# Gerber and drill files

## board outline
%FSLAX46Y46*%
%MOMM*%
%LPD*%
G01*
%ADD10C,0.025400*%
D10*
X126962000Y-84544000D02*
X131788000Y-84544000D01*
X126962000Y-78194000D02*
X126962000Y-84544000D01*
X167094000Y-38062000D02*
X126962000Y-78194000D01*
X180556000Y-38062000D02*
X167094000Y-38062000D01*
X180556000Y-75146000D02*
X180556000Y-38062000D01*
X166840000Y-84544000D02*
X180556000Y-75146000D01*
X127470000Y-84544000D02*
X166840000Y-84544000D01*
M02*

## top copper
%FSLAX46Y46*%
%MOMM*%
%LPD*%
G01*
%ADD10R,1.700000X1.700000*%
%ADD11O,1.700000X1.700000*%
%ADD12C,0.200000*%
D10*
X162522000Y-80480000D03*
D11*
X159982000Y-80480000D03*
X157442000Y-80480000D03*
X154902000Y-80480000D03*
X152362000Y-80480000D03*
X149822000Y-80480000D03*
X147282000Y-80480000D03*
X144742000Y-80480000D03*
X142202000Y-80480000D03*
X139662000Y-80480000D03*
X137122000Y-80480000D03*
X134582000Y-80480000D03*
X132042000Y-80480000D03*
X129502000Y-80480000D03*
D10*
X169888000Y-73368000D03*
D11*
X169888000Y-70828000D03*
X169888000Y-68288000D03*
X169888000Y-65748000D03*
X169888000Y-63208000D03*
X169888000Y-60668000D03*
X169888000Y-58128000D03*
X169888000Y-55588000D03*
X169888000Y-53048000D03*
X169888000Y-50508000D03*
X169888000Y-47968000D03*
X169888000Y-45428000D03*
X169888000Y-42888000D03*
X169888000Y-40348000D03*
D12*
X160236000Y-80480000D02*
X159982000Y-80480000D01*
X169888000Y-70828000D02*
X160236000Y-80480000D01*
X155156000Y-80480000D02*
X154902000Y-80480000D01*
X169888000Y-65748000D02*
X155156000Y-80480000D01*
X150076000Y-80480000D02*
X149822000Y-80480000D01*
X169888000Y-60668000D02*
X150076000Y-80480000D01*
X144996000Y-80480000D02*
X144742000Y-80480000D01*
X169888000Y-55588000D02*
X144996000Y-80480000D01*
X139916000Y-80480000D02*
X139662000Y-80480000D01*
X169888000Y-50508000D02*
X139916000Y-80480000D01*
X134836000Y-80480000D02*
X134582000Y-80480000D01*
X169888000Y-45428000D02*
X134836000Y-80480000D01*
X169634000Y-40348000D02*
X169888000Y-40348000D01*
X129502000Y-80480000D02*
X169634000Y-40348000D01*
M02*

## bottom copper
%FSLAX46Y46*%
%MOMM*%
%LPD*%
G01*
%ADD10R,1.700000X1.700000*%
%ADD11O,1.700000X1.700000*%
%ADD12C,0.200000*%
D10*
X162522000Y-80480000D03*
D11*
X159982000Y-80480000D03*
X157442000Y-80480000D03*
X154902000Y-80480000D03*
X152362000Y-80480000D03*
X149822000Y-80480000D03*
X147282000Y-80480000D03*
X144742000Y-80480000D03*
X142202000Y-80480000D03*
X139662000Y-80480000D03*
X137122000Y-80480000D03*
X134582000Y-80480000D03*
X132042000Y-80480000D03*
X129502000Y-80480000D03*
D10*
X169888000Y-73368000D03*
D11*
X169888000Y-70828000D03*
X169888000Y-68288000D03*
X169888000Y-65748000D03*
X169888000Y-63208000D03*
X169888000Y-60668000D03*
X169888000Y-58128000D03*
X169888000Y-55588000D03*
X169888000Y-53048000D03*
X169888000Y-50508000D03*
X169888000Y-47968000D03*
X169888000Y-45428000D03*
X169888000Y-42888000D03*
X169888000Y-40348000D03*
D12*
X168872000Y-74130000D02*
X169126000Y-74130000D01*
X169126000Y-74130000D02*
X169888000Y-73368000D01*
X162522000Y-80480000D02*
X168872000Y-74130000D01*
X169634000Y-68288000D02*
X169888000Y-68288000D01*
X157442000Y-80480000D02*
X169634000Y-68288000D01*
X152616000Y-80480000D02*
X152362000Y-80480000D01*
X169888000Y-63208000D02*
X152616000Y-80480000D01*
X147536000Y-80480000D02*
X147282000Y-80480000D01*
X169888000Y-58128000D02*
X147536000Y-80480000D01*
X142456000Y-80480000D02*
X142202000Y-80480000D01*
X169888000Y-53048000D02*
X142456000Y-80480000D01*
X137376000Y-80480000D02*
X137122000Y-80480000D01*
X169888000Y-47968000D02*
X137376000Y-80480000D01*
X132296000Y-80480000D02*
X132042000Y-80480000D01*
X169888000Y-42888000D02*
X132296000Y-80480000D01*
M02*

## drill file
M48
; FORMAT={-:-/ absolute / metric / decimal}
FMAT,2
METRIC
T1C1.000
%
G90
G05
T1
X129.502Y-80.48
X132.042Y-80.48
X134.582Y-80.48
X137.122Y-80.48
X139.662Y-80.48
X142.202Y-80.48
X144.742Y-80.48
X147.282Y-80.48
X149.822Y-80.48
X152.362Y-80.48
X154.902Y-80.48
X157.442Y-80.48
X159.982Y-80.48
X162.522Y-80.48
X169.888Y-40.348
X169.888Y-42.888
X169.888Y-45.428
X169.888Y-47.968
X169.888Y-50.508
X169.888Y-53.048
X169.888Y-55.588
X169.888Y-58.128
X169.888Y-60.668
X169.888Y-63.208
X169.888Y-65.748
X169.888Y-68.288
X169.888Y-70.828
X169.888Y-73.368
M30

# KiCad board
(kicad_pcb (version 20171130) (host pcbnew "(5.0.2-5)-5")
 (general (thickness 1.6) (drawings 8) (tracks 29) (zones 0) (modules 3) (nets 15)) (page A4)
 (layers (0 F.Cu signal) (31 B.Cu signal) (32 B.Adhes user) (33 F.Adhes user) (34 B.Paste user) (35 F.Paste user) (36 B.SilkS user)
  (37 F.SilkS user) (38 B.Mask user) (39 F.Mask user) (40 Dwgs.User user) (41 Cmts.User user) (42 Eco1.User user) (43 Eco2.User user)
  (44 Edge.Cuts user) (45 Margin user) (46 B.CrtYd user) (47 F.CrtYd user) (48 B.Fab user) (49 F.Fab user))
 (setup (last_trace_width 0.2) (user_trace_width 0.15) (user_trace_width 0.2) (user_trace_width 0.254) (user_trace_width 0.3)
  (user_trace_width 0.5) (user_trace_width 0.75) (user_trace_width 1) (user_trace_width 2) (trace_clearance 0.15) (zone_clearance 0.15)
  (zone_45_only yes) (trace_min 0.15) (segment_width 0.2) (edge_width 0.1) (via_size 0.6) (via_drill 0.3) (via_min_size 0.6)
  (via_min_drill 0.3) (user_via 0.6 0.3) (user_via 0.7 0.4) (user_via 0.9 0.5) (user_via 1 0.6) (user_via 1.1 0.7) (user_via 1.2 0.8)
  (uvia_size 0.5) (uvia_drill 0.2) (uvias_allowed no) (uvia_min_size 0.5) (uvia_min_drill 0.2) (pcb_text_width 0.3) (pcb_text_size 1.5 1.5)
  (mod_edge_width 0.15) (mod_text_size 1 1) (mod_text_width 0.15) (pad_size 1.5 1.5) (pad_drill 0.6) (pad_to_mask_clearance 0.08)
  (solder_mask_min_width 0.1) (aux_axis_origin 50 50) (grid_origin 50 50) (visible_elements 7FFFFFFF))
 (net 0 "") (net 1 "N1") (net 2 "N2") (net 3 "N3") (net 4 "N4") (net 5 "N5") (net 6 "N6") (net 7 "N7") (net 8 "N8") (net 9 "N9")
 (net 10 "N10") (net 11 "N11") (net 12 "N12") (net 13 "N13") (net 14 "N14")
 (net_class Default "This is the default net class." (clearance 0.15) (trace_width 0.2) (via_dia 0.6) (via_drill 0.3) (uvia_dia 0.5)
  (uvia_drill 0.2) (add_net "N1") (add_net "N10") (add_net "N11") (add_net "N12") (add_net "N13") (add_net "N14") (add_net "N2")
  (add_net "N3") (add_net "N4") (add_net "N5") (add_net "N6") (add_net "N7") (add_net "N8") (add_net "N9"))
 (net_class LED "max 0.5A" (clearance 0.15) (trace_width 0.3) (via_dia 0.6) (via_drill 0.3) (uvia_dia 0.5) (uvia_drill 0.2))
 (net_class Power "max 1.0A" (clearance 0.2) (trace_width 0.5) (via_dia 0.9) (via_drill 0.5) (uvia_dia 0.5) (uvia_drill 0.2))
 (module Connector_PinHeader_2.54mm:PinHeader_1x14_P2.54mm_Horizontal (layer F.Cu) (at 162.522 80.48 270)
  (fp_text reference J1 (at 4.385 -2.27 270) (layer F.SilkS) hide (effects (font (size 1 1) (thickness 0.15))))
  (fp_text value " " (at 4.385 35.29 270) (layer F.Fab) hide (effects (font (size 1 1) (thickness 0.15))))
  (pad 1 thru_hole rect (at 0 0 270) (size 1.7 1.7) (drill 1) (layers *.Cu *.Mask) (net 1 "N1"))
  (pad 2 thru_hole oval (at 0 2.54 270) (size 1.7 1.7) (drill 1) (layers *.Cu *.Mask) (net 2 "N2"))
  (pad 3 thru_hole oval (at 0 5.08 270) (size 1.7 1.7) (drill 1) (layers *.Cu *.Mask) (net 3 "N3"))
  (pad 4 thru_hole oval (at 0 7.62 270) (size 1.7 1.7) (drill 1) (layers *.Cu *.Mask) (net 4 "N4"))
  (pad 5 thru_hole oval (at 0 10.16 270) (size 1.7 1.7) (drill 1) (layers *.Cu *.Mask) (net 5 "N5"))
  (pad 6 thru_hole oval (at 0 12.7 270) (size 1.7 1.7) (drill 1) (layers *.Cu *.Mask) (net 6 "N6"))
  (pad 7 thru_hole oval (at 0 15.24 270) (size 1.7 1.7) (drill 1) (layers *.Cu *.Mask) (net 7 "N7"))
  (pad 8 thru_hole oval (at 0 17.78 270) (size 1.7 1.7) (drill 1) (layers *.Cu *.Mask) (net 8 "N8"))
  (pad 9 thru_hole oval (at 0 20.32 270) (size 1.7 1.7) (drill 1) (layers *.Cu *.Mask) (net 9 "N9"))
  (pad 10 thru_hole oval (at 0 22.86 270) (size 1.7 1.7) (drill 1) (layers *.Cu *.Mask) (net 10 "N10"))
  (pad 11 thru_hole oval (at 0 25.4 270) (size 1.7 1.7) (drill 1) (layers *.Cu *.Mask) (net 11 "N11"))
  (pad 12 thru_hole oval (at 0 27.94 270) (size 1.7 1.7) (drill 1) (layers *.Cu *.Mask) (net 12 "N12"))
  (pad 13 thru_hole oval (at 0 30.48 270) (size 1.7 1.7) (drill 1) (layers *.Cu *.Mask) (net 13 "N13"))
  (pad 14 thru_hole oval (at 0 33.02 270) (size 1.7 1.7) (drill 1) (layers *.Cu *.Mask) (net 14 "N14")))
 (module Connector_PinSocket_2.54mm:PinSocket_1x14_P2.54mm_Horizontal (layer F.Cu) (at 169.888 73.368 180)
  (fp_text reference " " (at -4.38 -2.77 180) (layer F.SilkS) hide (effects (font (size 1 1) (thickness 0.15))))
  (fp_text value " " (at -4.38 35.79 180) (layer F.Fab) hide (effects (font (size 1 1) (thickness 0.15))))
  (pad 1 thru_hole rect (at 0 0 180) (size 1.7 1.7) (drill 1) (layers *.Cu *.Mask) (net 1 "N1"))
  (pad 2 thru_hole oval (at 0 2.54 180) (size 1.7 1.7) (drill 1) (layers *.Cu *.Mask) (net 2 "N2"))
  (pad 3 thru_hole oval (at 0 5.08 180) (size 1.7 1.7) (drill 1) (layers *.Cu *.Mask) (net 3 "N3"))
  (pad 4 thru_hole oval (at 0 7.62 180) (size 1.7 1.7) (drill 1) (layers *.Cu *.Mask) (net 4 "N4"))
  (pad 5 thru_hole oval (at 0 10.16 180) (size 1.7 1.7) (drill 1) (layers *.Cu *.Mask) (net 5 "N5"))
  (pad 6 thru_hole oval (at 0 12.7 180) (size 1.7 1.7) (drill 1) (layers *.Cu *.Mask) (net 6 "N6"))
  (pad 7 thru_hole oval (at 0 15.24 180) (size 1.7 1.7) (drill 1) (layers *.Cu *.Mask) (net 7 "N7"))
  (pad 8 thru_hole oval (at 0 17.78 180) (size 1.7 1.7) (drill 1) (layers *.Cu *.Mask) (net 8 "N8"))
  (pad 9 thru_hole oval (at 0 20.32 180) (size 1.7 1.7) (drill 1) (layers *.Cu *.Mask) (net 9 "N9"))
  (pad 10 thru_hole oval (at 0 22.86 180) (size 1.7 1.7) (drill 1) (layers *.Cu *.Mask) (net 10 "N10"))
  (pad 11 thru_hole oval (at 0 25.4 180) (size 1.7 1.7) (drill 1) (layers *.Cu *.Mask) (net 11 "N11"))
  (pad 12 thru_hole oval (at 0 27.94 180) (size 1.7 1.7) (drill 1) (layers *.Cu *.Mask) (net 12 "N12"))
  (pad 13 thru_hole oval (at 0 30.48 180) (size 1.7 1.7) (drill 1) (layers *.Cu *.Mask) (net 13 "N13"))
  (pad 14 thru_hole oval (at 0 33.02 180) (size 1.7 1.7) (drill 1) (layers *.Cu *.Mask) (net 14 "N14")))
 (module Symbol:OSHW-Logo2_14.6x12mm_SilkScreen (layer B.Cu) (at 151.346 69.812 180)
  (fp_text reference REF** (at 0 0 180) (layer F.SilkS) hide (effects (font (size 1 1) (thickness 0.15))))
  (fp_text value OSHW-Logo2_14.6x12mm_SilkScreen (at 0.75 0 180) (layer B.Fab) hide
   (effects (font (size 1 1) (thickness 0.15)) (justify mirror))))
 (gr_line (start 126.962 84.544) (end 131.788 84.544) (layer Edge.Cuts) (width 0.0254))
 (gr_line (start 126.962 78.194) (end 126.962 84.544) (layer Edge.Cuts) (width 0.0254))
 (gr_line (start 167.094 38.062) (end 126.962 78.194) (layer Edge.Cuts) (width 0.0254))
 (gr_line (start 180.556 38.062) (end 167.094 38.062) (layer Edge.Cuts) (width 0.0254))
 (gr_line (start 180.556 75.146) (end 180.556 38.062) (layer Edge.Cuts) (width 0.0254))
 (gr_line (start 166.84 84.544) (end 180.556 75.146) (layer Edge.Cuts) (width 0.0254))
 (gr_line (start 127.47 84.544) (end 166.84 84.544) (layer Edge.Cuts) (width 0.0254))
 (segment (start 168.872 74.13) (end 169.126 74.13) (width 0.2) (layer B.Cu) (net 1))
 (segment (start 169.126 74.13) (end 169.888 73.368) (width 0.2) (layer B.Cu) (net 1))
 (segment (start 162.522 80.48) (end 168.872 74.13) (width 0.2) (layer B.Cu) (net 1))
 (segment (start 160.236 80.48) (end 159.982 80.48) (width 0.2) (layer F.Cu) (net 2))
 (segment (start 169.888 70.828) (end 160.236 80.48) (width 0.2) (layer F.Cu) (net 2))
 (segment (start 169.634 68.288) (end 169.888 68.288) (width 0.2) (layer B.Cu) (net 3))
 (segment (start 157.442 80.48) (end 169.634 68.288) (width 0.2) (layer B.Cu) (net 3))
 (segment (start 155.156 80.48) (end 154.902 80.48) (width 0.2) (layer F.Cu) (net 4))
 (segment (start 169.888 65.748) (end 155.156 80.48) (width 0.2) (layer F.Cu) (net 4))
 (segment (start 152.616 80.48) (end 152.362 80.48) (width 0.2) (layer B.Cu) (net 5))
 (segment (start 169.888 63.208) (end 152.616 80.48) (width 0.2) (layer B.Cu) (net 5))
 (segment (start 150.076 80.48) (end 149.822 80.48) (width 0.2) (layer F.Cu) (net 6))
 (segment (start 169.888 60.668) (end 150.076 80.48) (width 0.2) (layer F.Cu) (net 6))
 (segment (start 147.536 80.48) (end 147.282 80.48) (width 0.2) (layer B.Cu) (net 7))
 (segment (start 169.888 58.128) (end 147.536 80.48) (width 0.2) (layer B.Cu) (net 7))
 (segment (start 144.996 80.48) (end 144.742 80.48) (width 0.2) (layer F.Cu) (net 8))
 (segment (start 169.888 55.588) (end 144.996 80.48) (width 0.2) (layer F.Cu) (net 8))
 (segment (start 142.456 80.48) (end 142.202 80.48) (width 0.2) (layer B.Cu) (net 9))
 (segment (start 169.888 53.048) (end 142.456 80.48) (width 0.2) (layer B.Cu) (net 9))
 (segment (start 139.916 80.48) (end 139.662 80.48) (width 0.2) (layer F.Cu) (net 10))
 (segment (start 169.888 50.508) (end 139.916 80.48) (width 0.2) (layer F.Cu) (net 10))
 (segment (start 137.376 80.48) (end 137.122 80.48) (width 0.2) (layer B.Cu) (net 11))
 (segment (start 169.888 47.968) (end 137.376 80.48) (width 0.2) (layer B.Cu) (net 11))
 (segment (start 134.836 80.48) (end 134.582 80.48) (width 0.2) (layer F.Cu) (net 12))
 (segment (start 169.888 45.428) (end 134.836 80.48) (width 0.2) (layer F.Cu) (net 12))
 (segment (start 132.296 80.48) (end 132.042 80.48) (width 0.2) (layer B.Cu) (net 13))
 (segment (start 169.888 42.888) (end 132.296 80.48) (width 0.2) (layer B.Cu) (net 13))
 (segment (start 169.634 40.348) (end 169.888 40.348) (width 0.2) (layer F.Cu) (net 14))
 (segment (start 129.502 80.48) (end 169.634 40.348) (width 0.2) (layer F.Cu) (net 14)))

